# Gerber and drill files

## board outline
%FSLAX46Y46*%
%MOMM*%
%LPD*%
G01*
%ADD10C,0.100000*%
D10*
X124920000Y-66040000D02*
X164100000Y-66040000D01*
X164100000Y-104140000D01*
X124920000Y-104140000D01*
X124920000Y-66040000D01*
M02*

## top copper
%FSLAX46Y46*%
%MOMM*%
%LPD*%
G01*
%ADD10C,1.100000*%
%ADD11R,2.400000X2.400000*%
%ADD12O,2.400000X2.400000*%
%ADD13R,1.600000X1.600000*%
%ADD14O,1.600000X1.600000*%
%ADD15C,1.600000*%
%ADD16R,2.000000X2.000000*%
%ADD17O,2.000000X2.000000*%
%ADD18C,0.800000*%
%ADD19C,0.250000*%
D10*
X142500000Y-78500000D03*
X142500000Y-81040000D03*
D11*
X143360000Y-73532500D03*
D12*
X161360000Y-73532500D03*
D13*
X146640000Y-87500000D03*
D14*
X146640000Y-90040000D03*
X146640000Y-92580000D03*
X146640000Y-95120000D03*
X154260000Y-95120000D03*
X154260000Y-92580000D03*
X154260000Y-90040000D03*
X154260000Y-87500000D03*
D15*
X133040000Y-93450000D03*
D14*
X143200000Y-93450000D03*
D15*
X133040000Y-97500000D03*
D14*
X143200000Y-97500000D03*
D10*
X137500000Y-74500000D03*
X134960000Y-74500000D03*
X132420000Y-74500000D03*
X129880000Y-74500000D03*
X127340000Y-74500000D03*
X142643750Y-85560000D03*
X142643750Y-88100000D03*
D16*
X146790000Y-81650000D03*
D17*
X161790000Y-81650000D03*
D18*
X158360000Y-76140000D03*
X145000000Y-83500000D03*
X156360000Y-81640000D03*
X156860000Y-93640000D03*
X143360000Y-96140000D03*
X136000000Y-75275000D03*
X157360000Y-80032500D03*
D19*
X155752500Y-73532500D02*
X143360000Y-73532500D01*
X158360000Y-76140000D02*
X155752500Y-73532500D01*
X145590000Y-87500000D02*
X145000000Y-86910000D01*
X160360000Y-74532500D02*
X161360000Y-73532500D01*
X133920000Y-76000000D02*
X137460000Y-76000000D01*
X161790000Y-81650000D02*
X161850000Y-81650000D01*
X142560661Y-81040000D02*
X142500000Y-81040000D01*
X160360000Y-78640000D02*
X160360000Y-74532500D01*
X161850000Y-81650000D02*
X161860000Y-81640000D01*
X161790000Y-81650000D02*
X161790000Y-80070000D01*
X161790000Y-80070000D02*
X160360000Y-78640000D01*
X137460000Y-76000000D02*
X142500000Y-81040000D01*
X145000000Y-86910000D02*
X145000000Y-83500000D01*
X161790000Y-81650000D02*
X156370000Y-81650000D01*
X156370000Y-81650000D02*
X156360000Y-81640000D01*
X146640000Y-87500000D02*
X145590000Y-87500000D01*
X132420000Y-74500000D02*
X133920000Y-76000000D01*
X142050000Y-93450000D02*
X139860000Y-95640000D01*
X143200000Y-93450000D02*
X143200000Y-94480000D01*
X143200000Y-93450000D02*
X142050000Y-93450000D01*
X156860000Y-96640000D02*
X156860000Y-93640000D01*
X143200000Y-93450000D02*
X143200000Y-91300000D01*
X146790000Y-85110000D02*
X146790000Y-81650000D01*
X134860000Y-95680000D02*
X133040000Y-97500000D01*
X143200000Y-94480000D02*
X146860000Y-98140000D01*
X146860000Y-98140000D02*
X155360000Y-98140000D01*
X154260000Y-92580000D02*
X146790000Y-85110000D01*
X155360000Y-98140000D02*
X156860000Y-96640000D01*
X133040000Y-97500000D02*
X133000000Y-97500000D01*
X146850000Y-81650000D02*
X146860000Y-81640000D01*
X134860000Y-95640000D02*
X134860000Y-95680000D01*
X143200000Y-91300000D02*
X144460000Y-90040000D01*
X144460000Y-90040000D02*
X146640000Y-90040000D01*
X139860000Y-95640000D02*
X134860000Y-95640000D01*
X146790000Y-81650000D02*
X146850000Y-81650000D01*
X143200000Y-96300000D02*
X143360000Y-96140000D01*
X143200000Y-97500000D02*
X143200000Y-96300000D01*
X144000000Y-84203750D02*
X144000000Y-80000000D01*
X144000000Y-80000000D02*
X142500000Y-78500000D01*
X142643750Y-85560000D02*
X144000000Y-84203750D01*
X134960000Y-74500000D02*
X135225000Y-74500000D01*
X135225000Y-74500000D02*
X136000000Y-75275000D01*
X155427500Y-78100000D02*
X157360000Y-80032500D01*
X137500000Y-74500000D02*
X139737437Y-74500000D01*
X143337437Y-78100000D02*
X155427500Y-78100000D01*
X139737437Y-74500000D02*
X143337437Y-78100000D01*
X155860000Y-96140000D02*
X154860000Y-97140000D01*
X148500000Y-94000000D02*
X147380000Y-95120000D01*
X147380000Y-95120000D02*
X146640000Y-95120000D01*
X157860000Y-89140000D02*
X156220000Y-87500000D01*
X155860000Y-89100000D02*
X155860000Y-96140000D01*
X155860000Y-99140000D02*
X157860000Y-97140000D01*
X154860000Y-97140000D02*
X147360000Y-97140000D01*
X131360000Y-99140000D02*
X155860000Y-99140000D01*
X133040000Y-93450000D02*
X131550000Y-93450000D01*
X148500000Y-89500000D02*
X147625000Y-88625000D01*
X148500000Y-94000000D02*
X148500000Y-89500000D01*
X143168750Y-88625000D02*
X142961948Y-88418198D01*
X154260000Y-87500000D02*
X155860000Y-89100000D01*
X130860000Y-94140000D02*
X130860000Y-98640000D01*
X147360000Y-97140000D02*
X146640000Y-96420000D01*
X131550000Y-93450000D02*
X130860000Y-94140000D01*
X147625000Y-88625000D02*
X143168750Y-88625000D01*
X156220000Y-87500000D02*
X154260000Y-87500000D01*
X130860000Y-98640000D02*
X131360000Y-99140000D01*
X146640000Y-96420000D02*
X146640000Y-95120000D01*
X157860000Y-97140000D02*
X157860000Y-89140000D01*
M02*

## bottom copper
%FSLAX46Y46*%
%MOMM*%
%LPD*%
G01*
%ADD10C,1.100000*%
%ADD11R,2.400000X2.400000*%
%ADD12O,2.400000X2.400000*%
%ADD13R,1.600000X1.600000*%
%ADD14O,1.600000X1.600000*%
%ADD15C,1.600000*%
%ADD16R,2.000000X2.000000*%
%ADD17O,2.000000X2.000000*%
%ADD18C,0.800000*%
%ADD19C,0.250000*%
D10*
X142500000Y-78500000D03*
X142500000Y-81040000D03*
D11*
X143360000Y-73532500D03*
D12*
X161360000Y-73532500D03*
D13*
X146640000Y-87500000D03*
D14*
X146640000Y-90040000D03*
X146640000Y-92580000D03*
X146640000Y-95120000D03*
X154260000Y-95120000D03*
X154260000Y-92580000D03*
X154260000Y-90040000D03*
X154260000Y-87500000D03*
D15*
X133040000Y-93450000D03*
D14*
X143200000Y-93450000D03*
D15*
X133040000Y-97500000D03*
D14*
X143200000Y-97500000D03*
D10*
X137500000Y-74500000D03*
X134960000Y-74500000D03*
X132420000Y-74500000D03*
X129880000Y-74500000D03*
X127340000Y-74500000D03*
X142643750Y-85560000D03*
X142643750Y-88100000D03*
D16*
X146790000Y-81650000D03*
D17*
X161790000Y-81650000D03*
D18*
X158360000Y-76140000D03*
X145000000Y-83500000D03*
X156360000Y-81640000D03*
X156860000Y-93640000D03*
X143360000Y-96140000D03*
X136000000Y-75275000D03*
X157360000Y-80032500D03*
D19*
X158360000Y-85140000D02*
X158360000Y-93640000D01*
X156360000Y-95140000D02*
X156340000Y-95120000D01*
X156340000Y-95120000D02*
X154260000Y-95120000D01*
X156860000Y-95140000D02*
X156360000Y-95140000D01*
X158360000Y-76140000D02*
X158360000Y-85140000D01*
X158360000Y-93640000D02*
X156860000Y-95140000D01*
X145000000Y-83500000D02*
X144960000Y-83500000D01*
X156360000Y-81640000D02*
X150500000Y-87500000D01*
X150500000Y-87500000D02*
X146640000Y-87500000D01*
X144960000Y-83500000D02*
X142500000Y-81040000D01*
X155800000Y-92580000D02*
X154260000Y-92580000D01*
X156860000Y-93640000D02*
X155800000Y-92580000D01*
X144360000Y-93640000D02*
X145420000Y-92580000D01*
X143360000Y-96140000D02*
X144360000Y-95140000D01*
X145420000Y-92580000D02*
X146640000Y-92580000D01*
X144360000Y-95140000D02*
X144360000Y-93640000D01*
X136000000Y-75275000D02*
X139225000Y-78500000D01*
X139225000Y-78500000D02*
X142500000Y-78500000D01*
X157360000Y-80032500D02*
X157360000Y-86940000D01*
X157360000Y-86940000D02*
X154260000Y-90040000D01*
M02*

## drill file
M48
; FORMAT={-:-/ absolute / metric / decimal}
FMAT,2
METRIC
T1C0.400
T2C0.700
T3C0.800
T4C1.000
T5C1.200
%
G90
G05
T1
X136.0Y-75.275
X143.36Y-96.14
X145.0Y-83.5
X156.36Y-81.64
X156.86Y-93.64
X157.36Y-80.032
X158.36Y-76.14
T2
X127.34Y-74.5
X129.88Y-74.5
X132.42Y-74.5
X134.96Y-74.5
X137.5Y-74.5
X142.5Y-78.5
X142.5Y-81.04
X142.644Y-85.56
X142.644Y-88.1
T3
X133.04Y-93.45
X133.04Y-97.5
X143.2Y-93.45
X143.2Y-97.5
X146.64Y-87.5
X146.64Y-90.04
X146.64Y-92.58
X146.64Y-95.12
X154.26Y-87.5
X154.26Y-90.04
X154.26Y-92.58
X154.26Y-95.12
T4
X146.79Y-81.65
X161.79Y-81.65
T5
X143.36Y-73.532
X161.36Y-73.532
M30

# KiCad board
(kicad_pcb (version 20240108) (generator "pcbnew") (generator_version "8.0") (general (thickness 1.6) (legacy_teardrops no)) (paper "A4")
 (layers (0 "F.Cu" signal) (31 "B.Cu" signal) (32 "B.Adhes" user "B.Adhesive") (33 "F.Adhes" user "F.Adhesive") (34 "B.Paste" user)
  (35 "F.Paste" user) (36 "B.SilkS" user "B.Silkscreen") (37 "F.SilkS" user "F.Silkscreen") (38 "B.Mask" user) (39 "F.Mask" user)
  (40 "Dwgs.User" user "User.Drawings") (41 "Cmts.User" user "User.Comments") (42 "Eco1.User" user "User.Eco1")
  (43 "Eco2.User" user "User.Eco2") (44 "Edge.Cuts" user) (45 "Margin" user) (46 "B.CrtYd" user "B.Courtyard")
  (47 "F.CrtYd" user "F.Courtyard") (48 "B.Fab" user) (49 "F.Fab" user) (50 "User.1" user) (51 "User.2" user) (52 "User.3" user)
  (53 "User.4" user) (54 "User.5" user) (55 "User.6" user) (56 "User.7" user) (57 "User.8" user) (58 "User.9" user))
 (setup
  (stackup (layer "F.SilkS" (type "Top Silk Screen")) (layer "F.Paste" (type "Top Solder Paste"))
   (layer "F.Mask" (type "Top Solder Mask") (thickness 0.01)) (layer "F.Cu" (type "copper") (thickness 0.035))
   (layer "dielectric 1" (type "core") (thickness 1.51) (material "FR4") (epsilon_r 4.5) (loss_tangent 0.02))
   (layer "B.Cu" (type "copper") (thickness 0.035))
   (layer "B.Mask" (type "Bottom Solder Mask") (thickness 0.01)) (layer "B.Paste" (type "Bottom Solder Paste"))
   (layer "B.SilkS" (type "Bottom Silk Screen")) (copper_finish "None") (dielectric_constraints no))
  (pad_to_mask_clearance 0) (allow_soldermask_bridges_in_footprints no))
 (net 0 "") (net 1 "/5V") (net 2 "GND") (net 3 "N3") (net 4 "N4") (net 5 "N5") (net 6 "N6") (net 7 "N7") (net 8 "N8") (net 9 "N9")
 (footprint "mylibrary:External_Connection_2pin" (layer "F.Cu") (at 142.5 81.04)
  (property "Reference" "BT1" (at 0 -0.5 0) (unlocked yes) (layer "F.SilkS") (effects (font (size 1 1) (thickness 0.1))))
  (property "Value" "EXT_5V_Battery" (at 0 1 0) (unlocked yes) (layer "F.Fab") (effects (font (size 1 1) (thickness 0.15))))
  (pad "1" thru_hole circle (at 0 -2.54) (size 1.1 1.1) (drill 0.7) (layers "*.Cu" "*.Mask") (remove_unused_layers no) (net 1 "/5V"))
  (pad "2" thru_hole circle (at 0 0) (size 1.1 1.1) (drill 0.7) (layers "*.Cu" "*.Mask") (remove_unused_layers no) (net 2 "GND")))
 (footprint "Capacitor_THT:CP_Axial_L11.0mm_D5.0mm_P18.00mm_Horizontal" (layer "F.Cu") (at 143.36 73.5325)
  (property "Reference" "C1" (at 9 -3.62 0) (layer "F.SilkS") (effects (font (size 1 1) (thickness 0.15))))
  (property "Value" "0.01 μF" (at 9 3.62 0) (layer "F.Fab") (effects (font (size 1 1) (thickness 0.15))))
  (pad "1" thru_hole rect (at 0 0) (size 2.4 2.4) (drill 1.2) (layers "*.Cu" "*.Mask") (remove_unused_layers no) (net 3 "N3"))
  (pad "2" thru_hole oval (at 18 0) (size 2.4 2.4) (drill 1.2) (layers "*.Cu" "*.Mask") (remove_unused_layers no) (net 2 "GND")))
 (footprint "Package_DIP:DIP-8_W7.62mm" (layer "F.Cu") (at 146.64 87.5)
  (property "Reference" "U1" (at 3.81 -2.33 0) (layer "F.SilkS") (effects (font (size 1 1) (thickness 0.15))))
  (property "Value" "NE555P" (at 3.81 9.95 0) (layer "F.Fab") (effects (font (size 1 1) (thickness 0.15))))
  (pad "1" thru_hole rect (at 0 0) (size 1.6 1.6) (drill 0.8) (layers "*.Cu" "*.Mask") (remove_unused_layers no) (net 2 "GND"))
  (pad "2" thru_hole oval (at 0 2.54) (size 1.6 1.6) (drill 0.8) (layers "*.Cu" "*.Mask") (remove_unused_layers no) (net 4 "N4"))
  (pad "3" thru_hole oval (at 0 5.08) (size 1.6 1.6) (drill 0.8) (layers "*.Cu" "*.Mask") (remove_unused_layers no) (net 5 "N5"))
  (pad "4" thru_hole oval (at 0 7.62) (size 1.6 1.6) (drill 0.8) (layers "*.Cu" "*.Mask") (remove_unused_layers no) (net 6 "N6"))
  (pad "5" thru_hole oval (at 7.62 7.62) (size 1.6 1.6) (drill 0.8) (layers "*.Cu" "*.Mask") (remove_unused_layers no) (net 3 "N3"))
  (pad "6" thru_hole oval (at 7.62 5.08) (size 1.6 1.6) (drill 0.8) (layers "*.Cu" "*.Mask") (remove_unused_layers no) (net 4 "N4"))
  (pad "7" thru_hole oval (at 7.62 2.54) (size 1.6 1.6) (drill 0.8) (layers "*.Cu" "*.Mask") (remove_unused_layers no) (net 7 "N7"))
  (pad "8" thru_hole oval (at 7.62 0) (size 1.6 1.6) (drill 0.8) (layers "*.Cu" "*.Mask") (remove_unused_layers no) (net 6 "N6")))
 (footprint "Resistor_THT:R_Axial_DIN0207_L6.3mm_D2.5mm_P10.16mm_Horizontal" (layer "F.Cu") (at 133.04 93.45)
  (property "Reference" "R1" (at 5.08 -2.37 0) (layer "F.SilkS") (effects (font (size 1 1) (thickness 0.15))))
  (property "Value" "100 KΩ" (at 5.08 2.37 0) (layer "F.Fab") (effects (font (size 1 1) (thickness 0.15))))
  (pad "1" thru_hole circle (at 0 0) (size 1.6 1.6) (drill 0.8) (layers "*.Cu" "*.Mask") (remove_unused_layers no) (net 6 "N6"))
  (pad "2" thru_hole oval (at 10.16 0) (size 1.6 1.6) (drill 0.8) (layers "*.Cu" "*.Mask") (remove_unused_layers no) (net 4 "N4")))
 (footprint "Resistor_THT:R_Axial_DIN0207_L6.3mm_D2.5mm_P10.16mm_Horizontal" (layer "F.Cu") (at 133.04 97.5)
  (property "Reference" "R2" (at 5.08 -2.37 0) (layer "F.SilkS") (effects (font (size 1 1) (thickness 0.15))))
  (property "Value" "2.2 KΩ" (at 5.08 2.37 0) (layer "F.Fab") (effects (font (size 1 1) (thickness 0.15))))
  (pad "1" thru_hole circle (at 0 0) (size 1.6 1.6) (drill 0.8) (layers "*.Cu" "*.Mask") (remove_unused_layers no) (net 4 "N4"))
  (pad "2" thru_hole oval (at 10.16 0) (size 1.6 1.6) (drill 0.8) (layers "*.Cu" "*.Mask") (remove_unused_layers no) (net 5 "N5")))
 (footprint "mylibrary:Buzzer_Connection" (layer "F.Cu") (at 132.42 74.5 -90)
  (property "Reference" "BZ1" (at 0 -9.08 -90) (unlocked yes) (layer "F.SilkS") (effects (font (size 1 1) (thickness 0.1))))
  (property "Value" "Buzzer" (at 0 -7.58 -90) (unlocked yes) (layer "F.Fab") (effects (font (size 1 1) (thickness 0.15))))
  (pad "1" thru_hole circle (at 0 -5.08 270) (size 1.1 1.1) (drill 0.7) (layers "*.Cu" "*.Mask") (remove_unused_layers no) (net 7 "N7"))
  (pad "2" thru_hole circle (at 0 -2.54 270) (size 1.1 1.1) (drill 0.7) (layers "*.Cu" "*.Mask") (remove_unused_layers no) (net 1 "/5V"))
  (pad "3" thru_hole circle (at 0 0 270) (size 1.1 1.1) (drill 0.7) (layers "*.Cu" "*.Mask") (remove_unused_layers no) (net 2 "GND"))
  (pad "4" thru_hole circle (at 0 2.54 270) (size 1.1 1.1) (drill 0.7) (layers "*.Cu" "*.Mask") (remove_unused_layers no) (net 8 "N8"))
  (pad "5" thru_hole circle (at 0 5.08 270) (size 1.1 1.1) (drill 0.7) (layers "*.Cu" "*.Mask") (remove_unused_layers no) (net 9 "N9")))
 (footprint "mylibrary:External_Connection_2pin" (layer "F.Cu") (at 142.64375 88.1)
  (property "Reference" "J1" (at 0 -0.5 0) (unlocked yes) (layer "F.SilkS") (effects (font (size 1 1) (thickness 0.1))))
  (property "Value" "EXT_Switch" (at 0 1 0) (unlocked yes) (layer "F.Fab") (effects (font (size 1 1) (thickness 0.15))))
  (pad "1" thru_hole circle (at 0 -2.54) (size 1.1 1.1) (drill 0.7) (layers "*.Cu" "*.Mask") (remove_unused_layers no) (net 1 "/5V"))
  (pad "2" thru_hole circle (at 0 0) (size 1.1 1.1) (drill 0.7) (layers "*.Cu" "*.Mask") (remove_unused_layers no) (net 6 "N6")))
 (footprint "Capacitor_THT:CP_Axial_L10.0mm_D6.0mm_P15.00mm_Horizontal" (layer "F.Cu") (at 146.79 81.65)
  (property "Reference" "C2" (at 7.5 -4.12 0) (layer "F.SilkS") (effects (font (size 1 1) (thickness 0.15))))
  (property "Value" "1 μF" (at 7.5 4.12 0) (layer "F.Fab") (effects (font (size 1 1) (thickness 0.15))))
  (pad "1" thru_hole rect (at 0 0) (size 2 2) (drill 1) (layers "*.Cu" "*.Mask") (remove_unused_layers no) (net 4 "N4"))
  (pad "2" thru_hole oval (at 15 0) (size 2 2) (drill 1) (layers "*.Cu" "*.Mask") (remove_unused_layers no) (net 2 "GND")))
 (gr_rect (start 124.92 66.04) (end 164.1 104.14) (locked yes) (stroke (width 0.1) (type default)) (fill none) (layer "Edge.Cuts"))
 (segment (start 155.7525 73.5325) (end 143.36 73.5325) (width 0.25) (layer "F.Cu") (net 3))
 (segment (start 158.36 76.14) (end 155.7525 73.5325) (width 0.25) (layer "F.Cu") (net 3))
 (via (at 158.36 76.14) (size 0.8) (drill 0.4) (layers "F.Cu" "B.Cu") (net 3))
 (segment (start 158.36 85.14) (end 158.36 93.64) (width 0.25) (layer "B.Cu") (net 3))
 (segment (start 156.36 95.14) (end 156.34 95.12) (width 0.25) (layer "B.Cu") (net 3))
 (segment (start 156.34 95.12) (end 154.26 95.12) (width 0.25) (layer "B.Cu") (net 3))
 (segment (start 156.86 95.14) (end 156.36 95.14) (width 0.25) (layer "B.Cu") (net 3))
 (segment (start 158.36 76.14) (end 158.36 85.14) (width 0.25) (layer "B.Cu") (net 3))
 (segment (start 158.36 93.64) (end 156.86 95.14) (width 0.25) (layer "B.Cu") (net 3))
 (segment (start 145.59 87.5) (end 145 86.91) (width 0.25) (layer "F.Cu") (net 2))
 (segment (start 160.36 74.5325) (end 161.36 73.5325) (width 0.25) (layer "F.Cu") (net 2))
 (segment (start 133.92 76) (end 137.46 76) (width 0.25) (layer "F.Cu") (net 2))
 (segment (start 161.79 81.65) (end 161.85 81.65) (width 0.25) (layer "F.Cu") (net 2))
 (segment (start 142.560661 81.04) (end 142.5 81.04) (width 0.25) (layer "F.Cu") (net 2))
 (segment (start 160.36 78.64) (end 160.36 74.5325) (width 0.25) (layer "F.Cu") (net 2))
 (segment (start 161.85 81.65) (end 161.86 81.64) (width 0.25) (layer "F.Cu") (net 2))
 (segment (start 161.79 81.65) (end 161.79 80.07) (width 0.25) (layer "F.Cu") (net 2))
 (segment (start 161.79 80.07) (end 160.36 78.64) (width 0.25) (layer "F.Cu") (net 2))
 (segment (start 137.46 76) (end 142.5 81.04) (width 0.25) (layer "F.Cu") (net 2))
 (segment (start 145 86.91) (end 145 83.5) (width 0.25) (layer "F.Cu") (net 2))
 (segment (start 161.79 81.65) (end 156.37 81.65) (width 0.25) (layer "F.Cu") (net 2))
 (segment (start 156.37 81.65) (end 156.36 81.64) (width 0.25) (layer "F.Cu") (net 2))
 (segment (start 146.64 87.5) (end 145.59 87.5) (width 0.25) (layer "F.Cu") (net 2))
 (segment (start 132.42 74.5) (end 133.92 76) (width 0.25) (layer "F.Cu") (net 2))
 (via (at 145 83.5) (size 0.8) (drill 0.4) (layers "F.Cu" "B.Cu") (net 2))
 (via (at 156.36 81.64) (size 0.8) (drill 0.4) (layers "F.Cu" "B.Cu") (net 2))
 (segment (start 145 83.5) (end 144.96 83.5) (width 0.25) (layer "B.Cu") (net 2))
 (segment (start 156.36 81.64) (end 150.5 87.5) (width 0.25) (layer "B.Cu") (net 2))
 (segment (start 150.5 87.5) (end 146.64 87.5) (width 0.25) (layer "B.Cu") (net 2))
 (segment (start 144.96 83.5) (end 142.5 81.04) (width 0.25) (layer "B.Cu") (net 2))
 (segment (start 142.05 93.45) (end 139.86 95.64) (width 0.25) (layer "F.Cu") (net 4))
 (segment (start 143.2 93.45) (end 143.2 94.48) (width 0.25) (layer "F.Cu") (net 4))
 (segment (start 143.2 93.45) (end 142.05 93.45) (width 0.25) (layer "F.Cu") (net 4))
 (segment (start 156.86 96.64) (end 156.86 93.64) (width 0.25) (layer "F.Cu") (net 4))
 (segment (start 143.2 93.45) (end 143.2 91.3) (width 0.25) (layer "F.Cu") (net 4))
 (segment (start 146.79 85.11) (end 146.79 81.65) (width 0.25) (layer "F.Cu") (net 4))
 (segment (start 134.86 95.68) (end 133.04 97.5) (width 0.25) (layer "F.Cu") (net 4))
 (segment (start 143.2 94.48) (end 146.86 98.14) (width 0.25) (layer "F.Cu") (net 4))
 (segment (start 146.86 98.14) (end 155.36 98.14) (width 0.25) (layer "F.Cu") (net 4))
 (segment (start 154.26 92.58) (end 146.79 85.11) (width 0.25) (layer "F.Cu") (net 4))
 (segment (start 155.36 98.14) (end 156.86 96.64) (width 0.25) (layer "F.Cu") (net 4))
 (segment (start 133.04 97.5) (end 133 97.5) (width 0.25) (layer "F.Cu") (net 4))
 (segment (start 146.85 81.65) (end 146.86 81.64) (width 0.25) (layer "F.Cu") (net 4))
 (segment (start 134.86 95.64) (end 134.86 95.68) (width 0.25) (layer "F.Cu") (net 4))
 (segment (start 143.2 91.3) (end 144.46 90.04) (width 0.25) (layer "F.Cu") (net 4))
 (segment (start 144.46 90.04) (end 146.64 90.04) (width 0.25) (layer "F.Cu") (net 4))
 (segment (start 139.86 95.64) (end 134.86 95.64) (width 0.25) (layer "F.Cu") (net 4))
 (segment (start 146.79 81.65) (end 146.85 81.65) (width 0.25) (layer "F.Cu") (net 4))
 (via (at 156.86 93.64) (size 0.8) (drill 0.4) (layers "F.Cu" "B.Cu") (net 4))
 (segment (start 155.8 92.58) (end 154.26 92.58) (width 0.25) (layer "B.Cu") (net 4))
 (segment (start 156.86 93.64) (end 155.8 92.58) (width 0.25) (layer "B.Cu") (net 4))
 (segment (start 143.2 96.3) (end 143.36 96.14) (width 0.25) (layer "F.Cu") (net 5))
 (segment (start 143.2 97.5) (end 143.2 96.3) (width 0.25) (layer "F.Cu") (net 5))
 (via (at 143.36 96.14) (size 0.8) (drill 0.4) (layers "F.Cu" "B.Cu") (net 5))
 (segment (start 144.36 93.64) (end 145.42 92.58) (width 0.25) (layer "B.Cu") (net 5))
 (segment (start 143.36 96.14) (end 144.36 95.14) (width 0.25) (layer "B.Cu") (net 5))
 (segment (start 145.42 92.58) (end 146.64 92.58) (width 0.25) (layer "B.Cu") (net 5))
 (segment (start 144.36 95.14) (end 144.36 93.64) (width 0.25) (layer "B.Cu") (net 5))
 (segment (start 144 84.20375) (end 144 80) (width 0.25) (layer "F.Cu") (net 1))
 (segment (start 144 80) (end 142.5 78.5) (width 0.25) (layer "F.Cu") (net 1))
 (segment (start 142.64375 85.56) (end 144 84.20375) (width 0.25) (layer "F.Cu") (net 1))
 (segment (start 134.96 74.5) (end 135.225 74.5) (width 0.25) (layer "F.Cu") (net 1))
 (segment (start 135.225 74.5) (end 136 75.275) (width 0.25) (layer "F.Cu") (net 1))
 (via (at 136 75.275) (size 0.8) (drill 0.4) (layers "F.Cu" "B.Cu") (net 1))
 (segment (start 136 75.275) (end 139.225 78.5) (width 0.25) (layer "B.Cu") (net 1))
 (segment (start 139.225 78.5) (end 142.5 78.5) (width 0.25) (layer "B.Cu") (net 1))
 (segment (start 155.4275 78.1) (end 157.36 80.0325) (width 0.25) (layer "F.Cu") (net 7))
 (segment (start 137.5 74.5) (end 139.737437 74.5) (width 0.25) (layer "F.Cu") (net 7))
 (segment (start 143.337437 78.1) (end 155.4275 78.1) (width 0.25) (layer "F.Cu") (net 7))
 (segment (start 139.737437 74.5) (end 143.337437 78.1) (width 0.25) (layer "F.Cu") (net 7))
 (via (at 157.36 80.0325) (size 0.8) (drill 0.4) (layers "F.Cu" "B.Cu") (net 7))
 (segment (start 157.36 80.0325) (end 157.36 86.94) (width 0.25) (layer "B.Cu") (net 7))
 (segment (start 157.36 86.94) (end 154.26 90.04) (width 0.25) (layer "B.Cu") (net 7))
 (segment (start 155.86 96.14) (end 154.86 97.14) (width 0.25) (layer "F.Cu") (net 6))
 (segment (start 148.5 94) (end 147.38 95.12) (width 0.25) (layer "F.Cu") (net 6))
 (segment (start 147.38 95.12) (end 146.64 95.12) (width 0.25) (layer "F.Cu") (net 6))
 (segment (start 157.86 89.14) (end 156.22 87.5) (width 0.25) (layer "F.Cu") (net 6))
 (segment (start 155.86 89.1) (end 155.86 96.14) (width 0.25) (layer "F.Cu") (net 6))
 (segment (start 155.86 99.14) (end 157.86 97.14) (width 0.25) (layer "F.Cu") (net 6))
 (segment (start 154.86 97.14) (end 147.36 97.14) (width 0.25) (layer "F.Cu") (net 6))
 (segment (start 131.36 99.14) (end 155.86 99.14) (width 0.25) (layer "F.Cu") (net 6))
 (segment (start 133.04 93.45) (end 131.55 93.45) (width 0.25) (layer "F.Cu") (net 6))
 (segment (start 148.5 89.5) (end 147.625 88.625) (width 0.25) (layer "F.Cu") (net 6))
 (segment (start 148.5 94) (end 148.5 89.5) (width 0.25) (layer "F.Cu") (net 6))
 (segment (start 143.16875 88.625) (end 142.961948 88.418198) (width 0.25) (layer "F.Cu") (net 6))
 (segment (start 154.26 87.5) (end 155.86 89.1) (width 0.25) (layer "F.Cu") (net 6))
 (segment (start 130.86 94.14) (end 130.86 98.64) (width 0.25) (layer "F.Cu") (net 6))
 (segment (start 147.36 97.14) (end 146.64 96.42) (width 0.25) (layer "F.Cu") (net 6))
 (segment (start 131.55 93.45) (end 130.86 94.14) (width 0.25) (layer "F.Cu") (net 6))
 (segment (start 147.625 88.625) (end 143.16875 88.625) (width 0.25) (layer "F.Cu") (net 6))
 (segment (start 156.22 87.5) (end 154.26 87.5) (width 0.25) (layer "F.Cu") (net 6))
 (segment (start 130.86 98.64) (end 131.36 99.14) (width 0.25) (layer "F.Cu") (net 6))
 (segment (start 146.64 96.42) (end 146.64 95.12) (width 0.25) (layer "F.Cu") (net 6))
 (segment (start 157.86 97.14) (end 157.86 89.14) (width 0.25) (layer "F.Cu") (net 6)))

